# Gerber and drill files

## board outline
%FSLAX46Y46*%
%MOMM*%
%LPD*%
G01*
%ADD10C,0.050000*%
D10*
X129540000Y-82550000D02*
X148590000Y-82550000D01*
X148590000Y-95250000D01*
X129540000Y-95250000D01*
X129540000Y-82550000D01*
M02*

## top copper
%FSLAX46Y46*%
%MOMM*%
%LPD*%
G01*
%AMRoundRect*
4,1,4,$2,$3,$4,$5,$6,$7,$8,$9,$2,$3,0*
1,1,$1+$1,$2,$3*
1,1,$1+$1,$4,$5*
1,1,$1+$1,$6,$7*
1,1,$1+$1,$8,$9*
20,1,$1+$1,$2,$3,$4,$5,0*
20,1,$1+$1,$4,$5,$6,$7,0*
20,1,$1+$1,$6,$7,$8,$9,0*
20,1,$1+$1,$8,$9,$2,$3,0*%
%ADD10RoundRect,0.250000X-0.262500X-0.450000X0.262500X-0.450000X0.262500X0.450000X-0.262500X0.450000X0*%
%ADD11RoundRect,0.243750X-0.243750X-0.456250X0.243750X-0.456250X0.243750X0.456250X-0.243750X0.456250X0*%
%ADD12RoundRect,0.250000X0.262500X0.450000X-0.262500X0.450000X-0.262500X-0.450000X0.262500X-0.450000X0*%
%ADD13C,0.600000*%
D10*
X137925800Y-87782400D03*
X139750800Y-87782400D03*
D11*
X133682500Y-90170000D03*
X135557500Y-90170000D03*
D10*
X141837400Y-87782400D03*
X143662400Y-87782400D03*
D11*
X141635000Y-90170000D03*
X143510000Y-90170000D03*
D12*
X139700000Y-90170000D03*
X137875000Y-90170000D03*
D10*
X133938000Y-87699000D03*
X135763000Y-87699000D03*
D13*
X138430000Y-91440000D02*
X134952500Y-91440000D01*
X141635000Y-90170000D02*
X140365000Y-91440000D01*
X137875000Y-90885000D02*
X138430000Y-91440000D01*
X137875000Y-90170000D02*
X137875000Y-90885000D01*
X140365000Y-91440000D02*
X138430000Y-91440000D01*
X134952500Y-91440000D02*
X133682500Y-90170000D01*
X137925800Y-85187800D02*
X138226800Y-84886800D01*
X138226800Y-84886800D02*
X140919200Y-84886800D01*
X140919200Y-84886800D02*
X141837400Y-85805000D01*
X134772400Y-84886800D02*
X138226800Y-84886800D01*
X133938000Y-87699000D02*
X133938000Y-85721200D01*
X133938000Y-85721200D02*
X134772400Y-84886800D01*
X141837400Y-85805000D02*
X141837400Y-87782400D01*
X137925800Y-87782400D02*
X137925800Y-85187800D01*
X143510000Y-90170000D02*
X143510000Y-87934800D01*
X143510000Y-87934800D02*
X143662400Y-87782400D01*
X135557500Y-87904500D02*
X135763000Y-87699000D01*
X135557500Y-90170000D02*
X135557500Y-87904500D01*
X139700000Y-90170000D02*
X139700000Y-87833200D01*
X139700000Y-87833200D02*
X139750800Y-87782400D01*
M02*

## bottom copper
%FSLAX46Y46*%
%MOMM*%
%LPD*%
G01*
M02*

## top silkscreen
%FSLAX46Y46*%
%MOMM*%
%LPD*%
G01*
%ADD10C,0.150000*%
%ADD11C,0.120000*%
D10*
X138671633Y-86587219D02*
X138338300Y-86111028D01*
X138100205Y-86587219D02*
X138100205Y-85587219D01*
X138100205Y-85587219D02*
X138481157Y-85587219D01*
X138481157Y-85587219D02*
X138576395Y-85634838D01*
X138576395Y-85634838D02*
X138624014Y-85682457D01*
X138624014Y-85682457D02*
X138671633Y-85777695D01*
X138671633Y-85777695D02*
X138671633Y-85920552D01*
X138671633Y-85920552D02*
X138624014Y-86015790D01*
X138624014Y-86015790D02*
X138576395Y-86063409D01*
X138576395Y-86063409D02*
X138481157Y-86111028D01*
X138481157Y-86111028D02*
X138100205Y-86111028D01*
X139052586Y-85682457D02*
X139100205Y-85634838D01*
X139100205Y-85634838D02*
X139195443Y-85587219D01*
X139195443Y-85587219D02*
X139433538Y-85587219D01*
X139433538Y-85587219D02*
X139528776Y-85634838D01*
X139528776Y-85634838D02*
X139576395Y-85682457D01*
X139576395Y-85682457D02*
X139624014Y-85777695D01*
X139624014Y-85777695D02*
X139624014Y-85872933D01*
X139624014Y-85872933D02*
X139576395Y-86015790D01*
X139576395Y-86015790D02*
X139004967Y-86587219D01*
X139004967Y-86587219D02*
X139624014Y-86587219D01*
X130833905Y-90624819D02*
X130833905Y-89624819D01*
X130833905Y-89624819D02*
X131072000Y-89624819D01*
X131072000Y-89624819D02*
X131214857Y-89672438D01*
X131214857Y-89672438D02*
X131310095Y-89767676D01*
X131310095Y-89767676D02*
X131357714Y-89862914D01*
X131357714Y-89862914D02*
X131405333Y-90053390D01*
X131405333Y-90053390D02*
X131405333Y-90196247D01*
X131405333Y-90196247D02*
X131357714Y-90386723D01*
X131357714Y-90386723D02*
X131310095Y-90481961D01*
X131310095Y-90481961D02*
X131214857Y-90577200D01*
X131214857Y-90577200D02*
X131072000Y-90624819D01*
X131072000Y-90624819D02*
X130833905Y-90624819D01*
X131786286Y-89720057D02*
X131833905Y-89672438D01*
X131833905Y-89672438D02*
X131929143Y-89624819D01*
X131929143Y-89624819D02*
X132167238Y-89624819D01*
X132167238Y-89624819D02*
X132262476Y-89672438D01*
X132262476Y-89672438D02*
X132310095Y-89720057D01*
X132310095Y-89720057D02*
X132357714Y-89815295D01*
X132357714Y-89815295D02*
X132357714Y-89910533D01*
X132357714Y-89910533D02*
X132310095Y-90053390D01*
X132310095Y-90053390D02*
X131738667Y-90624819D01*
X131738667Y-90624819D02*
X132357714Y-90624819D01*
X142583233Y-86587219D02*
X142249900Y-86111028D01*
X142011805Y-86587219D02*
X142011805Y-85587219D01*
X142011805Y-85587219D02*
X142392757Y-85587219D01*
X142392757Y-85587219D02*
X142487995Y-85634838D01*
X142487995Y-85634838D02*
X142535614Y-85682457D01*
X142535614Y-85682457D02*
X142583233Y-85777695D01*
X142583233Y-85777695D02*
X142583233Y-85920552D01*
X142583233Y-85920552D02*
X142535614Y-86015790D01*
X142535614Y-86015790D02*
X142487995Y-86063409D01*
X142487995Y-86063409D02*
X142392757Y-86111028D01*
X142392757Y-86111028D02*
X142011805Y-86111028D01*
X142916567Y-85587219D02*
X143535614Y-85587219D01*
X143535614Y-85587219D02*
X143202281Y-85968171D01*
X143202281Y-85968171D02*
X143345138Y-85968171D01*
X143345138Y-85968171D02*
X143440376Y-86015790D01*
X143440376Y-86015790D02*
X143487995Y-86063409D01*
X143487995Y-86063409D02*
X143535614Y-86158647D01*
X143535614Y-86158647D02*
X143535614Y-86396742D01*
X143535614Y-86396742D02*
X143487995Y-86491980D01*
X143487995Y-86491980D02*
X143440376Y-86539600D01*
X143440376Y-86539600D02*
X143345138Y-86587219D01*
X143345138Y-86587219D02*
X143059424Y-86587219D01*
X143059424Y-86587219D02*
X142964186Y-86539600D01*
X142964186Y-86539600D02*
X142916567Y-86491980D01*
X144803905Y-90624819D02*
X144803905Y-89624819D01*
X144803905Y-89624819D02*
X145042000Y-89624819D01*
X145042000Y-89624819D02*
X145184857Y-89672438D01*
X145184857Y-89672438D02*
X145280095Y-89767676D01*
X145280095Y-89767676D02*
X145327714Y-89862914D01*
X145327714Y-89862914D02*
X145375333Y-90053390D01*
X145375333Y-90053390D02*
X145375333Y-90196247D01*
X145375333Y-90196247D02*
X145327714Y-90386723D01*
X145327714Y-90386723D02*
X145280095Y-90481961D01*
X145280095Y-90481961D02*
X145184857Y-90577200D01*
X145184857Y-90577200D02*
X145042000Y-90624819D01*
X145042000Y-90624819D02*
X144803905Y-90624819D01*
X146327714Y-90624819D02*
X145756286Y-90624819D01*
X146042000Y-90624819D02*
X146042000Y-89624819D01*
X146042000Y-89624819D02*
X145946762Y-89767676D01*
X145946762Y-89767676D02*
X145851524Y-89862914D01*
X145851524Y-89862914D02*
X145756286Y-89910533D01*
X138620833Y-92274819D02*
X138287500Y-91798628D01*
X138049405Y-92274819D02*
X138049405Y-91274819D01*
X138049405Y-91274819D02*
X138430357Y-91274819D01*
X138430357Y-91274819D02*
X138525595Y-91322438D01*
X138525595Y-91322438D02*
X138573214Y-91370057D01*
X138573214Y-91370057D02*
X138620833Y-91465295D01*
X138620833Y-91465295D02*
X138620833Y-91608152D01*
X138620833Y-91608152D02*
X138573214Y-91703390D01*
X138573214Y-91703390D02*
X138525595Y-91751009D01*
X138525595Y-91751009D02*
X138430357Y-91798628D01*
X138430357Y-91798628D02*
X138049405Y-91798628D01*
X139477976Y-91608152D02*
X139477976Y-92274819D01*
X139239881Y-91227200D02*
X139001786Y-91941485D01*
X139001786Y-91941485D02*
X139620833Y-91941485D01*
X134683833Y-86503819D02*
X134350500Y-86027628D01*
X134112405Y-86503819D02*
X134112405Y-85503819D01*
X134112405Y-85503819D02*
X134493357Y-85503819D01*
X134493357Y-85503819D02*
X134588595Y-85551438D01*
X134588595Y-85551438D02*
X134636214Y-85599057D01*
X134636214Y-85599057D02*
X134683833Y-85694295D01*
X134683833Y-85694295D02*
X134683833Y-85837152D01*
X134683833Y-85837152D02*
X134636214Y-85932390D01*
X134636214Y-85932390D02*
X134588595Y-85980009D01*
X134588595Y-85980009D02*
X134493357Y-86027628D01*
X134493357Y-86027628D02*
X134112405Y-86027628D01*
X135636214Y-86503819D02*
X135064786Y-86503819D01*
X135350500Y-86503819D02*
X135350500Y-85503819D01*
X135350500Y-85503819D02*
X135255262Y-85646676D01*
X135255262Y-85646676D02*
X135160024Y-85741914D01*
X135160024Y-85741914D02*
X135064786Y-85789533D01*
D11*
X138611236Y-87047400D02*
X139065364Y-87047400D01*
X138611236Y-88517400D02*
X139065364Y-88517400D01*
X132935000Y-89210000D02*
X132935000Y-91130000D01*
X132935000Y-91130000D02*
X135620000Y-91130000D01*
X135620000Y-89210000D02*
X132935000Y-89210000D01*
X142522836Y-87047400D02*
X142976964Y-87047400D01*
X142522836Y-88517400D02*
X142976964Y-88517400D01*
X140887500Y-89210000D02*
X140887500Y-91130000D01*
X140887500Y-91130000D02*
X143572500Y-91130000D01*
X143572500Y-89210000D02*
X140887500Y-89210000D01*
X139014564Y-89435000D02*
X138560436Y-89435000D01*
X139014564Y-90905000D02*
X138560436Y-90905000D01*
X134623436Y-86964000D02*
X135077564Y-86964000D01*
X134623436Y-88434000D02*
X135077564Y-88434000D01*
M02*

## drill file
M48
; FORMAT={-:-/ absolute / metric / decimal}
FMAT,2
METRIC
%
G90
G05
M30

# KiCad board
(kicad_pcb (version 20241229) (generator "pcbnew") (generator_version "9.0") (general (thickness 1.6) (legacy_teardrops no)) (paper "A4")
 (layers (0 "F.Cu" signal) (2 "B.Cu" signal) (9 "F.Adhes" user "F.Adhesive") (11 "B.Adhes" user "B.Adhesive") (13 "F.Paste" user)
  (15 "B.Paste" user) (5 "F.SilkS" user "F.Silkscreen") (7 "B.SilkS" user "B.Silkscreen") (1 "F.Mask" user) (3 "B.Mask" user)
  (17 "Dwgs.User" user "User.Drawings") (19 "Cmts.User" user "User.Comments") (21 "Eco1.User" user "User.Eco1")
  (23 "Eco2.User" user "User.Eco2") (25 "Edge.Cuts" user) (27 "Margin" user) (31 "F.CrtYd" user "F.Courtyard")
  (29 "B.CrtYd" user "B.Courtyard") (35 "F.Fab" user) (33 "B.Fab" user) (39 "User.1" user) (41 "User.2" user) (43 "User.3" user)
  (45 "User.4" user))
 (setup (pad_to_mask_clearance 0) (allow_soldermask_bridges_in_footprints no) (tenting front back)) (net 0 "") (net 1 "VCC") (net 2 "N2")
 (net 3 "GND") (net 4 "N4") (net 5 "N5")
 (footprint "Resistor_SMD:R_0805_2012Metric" (layer "F.Cu") (at 138.8383 87.7824)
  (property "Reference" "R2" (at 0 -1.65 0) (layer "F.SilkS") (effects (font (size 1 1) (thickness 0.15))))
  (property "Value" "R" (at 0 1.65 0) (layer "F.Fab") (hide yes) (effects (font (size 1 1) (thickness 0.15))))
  (fp_line (start -0.227064 -0.735) (end 0.227064 -0.735) (stroke (width 0.12) (type solid)) (layer "F.SilkS"))
  (fp_line (start -0.227064 0.735) (end 0.227064 0.735) (stroke (width 0.12) (type solid)) (layer "F.SilkS"))
  (pad "1" smd roundrect (at -0.9125 0) (size 1.025 1.4) (layers "F.Cu" "F.Mask" "F.Paste") (roundrect_rratio 0.243902) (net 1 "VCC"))
  (pad "2" smd roundrect (at 0.9125 0) (size 1.025 1.4) (layers "F.Cu" "F.Mask" "F.Paste") (roundrect_rratio 0.243902) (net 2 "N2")))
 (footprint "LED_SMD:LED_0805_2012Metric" (layer "F.Cu") (at 134.62 90.17)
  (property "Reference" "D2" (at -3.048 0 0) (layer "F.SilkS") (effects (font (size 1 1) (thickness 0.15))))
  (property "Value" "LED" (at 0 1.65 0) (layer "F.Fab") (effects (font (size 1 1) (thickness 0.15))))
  (fp_line (start -1.685 -0.96) (end -1.685 0.96) (stroke (width 0.12) (type solid)) (layer "F.SilkS"))
  (fp_line (start -1.685 0.96) (end 1 0.96) (stroke (width 0.12) (type solid)) (layer "F.SilkS"))
  (fp_line (start 1 -0.96) (end -1.685 -0.96) (stroke (width 0.12) (type solid)) (layer "F.SilkS"))
  (pad "1" smd roundrect (at -0.9375 0) (size 0.975 1.4) (layers "F.Cu" "F.Mask" "F.Paste") (roundrect_rratio 0.25) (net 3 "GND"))
  (pad "2" smd roundrect (at 0.9375 0) (size 0.975 1.4) (layers "F.Cu" "F.Mask" "F.Paste") (roundrect_rratio 0.25) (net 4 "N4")))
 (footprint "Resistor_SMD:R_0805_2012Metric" (layer "F.Cu") (at 142.7499 87.7824)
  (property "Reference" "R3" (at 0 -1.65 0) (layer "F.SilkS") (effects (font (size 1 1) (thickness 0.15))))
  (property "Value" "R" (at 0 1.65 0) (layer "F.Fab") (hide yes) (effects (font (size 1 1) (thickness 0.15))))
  (fp_line (start -0.227064 -0.735) (end 0.227064 -0.735) (stroke (width 0.12) (type solid)) (layer "F.SilkS"))
  (fp_line (start -0.227064 0.735) (end 0.227064 0.735) (stroke (width 0.12) (type solid)) (layer "F.SilkS"))
  (pad "1" smd roundrect (at -0.9125 0) (size 1.025 1.4) (layers "F.Cu" "F.Mask" "F.Paste") (roundrect_rratio 0.243902) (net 1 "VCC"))
  (pad "2" smd roundrect (at 0.9125 0) (size 1.025 1.4) (layers "F.Cu" "F.Mask" "F.Paste") (roundrect_rratio 0.243902) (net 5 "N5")))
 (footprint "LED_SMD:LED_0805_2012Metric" (layer "F.Cu") (at 142.5725 90.17)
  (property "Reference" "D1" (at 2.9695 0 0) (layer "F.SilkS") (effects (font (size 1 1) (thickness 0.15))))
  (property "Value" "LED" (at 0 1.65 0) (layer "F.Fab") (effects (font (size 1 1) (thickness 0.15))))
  (fp_line (start -1.685 -0.96) (end -1.685 0.96) (stroke (width 0.12) (type solid)) (layer "F.SilkS"))
  (fp_line (start -1.685 0.96) (end 1 0.96) (stroke (width 0.12) (type solid)) (layer "F.SilkS"))
  (fp_line (start 1 -0.96) (end -1.685 -0.96) (stroke (width 0.12) (type solid)) (layer "F.SilkS"))
  (pad "1" smd roundrect (at -0.9375 0) (size 0.975 1.4) (layers "F.Cu" "F.Mask" "F.Paste") (roundrect_rratio 0.25) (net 3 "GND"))
  (pad "2" smd roundrect (at 0.9375 0) (size 0.975 1.4) (layers "F.Cu" "F.Mask" "F.Paste") (roundrect_rratio 0.25) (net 5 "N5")))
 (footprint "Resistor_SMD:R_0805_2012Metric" (layer "F.Cu") (at 138.7875 90.17 180)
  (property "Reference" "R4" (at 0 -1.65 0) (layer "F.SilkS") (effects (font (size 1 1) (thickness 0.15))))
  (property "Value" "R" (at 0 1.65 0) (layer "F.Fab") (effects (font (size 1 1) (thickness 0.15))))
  (fp_line (start -0.227064 0.735) (end 0.227064 0.735) (stroke (width 0.12) (type solid)) (layer "F.SilkS"))
  (fp_line (start -0.227064 -0.735) (end 0.227064 -0.735) (stroke (width 0.12) (type solid)) (layer "F.SilkS"))
  (pad "1" smd roundrect (at -0.9125 0 180) (size 1.025 1.4) (layers "F.Cu" "F.Mask" "F.Paste") (roundrect_rratio 0.243902) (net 2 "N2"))
  (pad "2" smd roundrect (at 0.9125 0 180) (size 1.025 1.4) (layers "F.Cu" "F.Mask" "F.Paste") (roundrect_rratio 0.243902) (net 3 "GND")))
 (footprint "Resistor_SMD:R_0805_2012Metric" (layer "F.Cu") (at 134.8505 87.699)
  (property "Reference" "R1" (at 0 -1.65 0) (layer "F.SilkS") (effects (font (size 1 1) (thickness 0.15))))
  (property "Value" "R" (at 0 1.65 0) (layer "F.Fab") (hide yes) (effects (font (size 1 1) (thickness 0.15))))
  (fp_line (start -0.227064 -0.735) (end 0.227064 -0.735) (stroke (width 0.12) (type solid)) (layer "F.SilkS"))
  (fp_line (start -0.227064 0.735) (end 0.227064 0.735) (stroke (width 0.12) (type solid)) (layer "F.SilkS"))
  (pad "1" smd roundrect (at -0.9125 0) (size 1.025 1.4) (layers "F.Cu" "F.Mask" "F.Paste") (roundrect_rratio 0.243902) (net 1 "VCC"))
  (pad "2" smd roundrect (at 0.9125 0) (size 1.025 1.4) (layers "F.Cu" "F.Mask" "F.Paste") (roundrect_rratio 0.243902) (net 4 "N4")))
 (gr_rect (start 129.54 82.55) (end 148.59 95.25) (stroke (width 0.05) (type default)) (fill no) (layer "Edge.Cuts"))
 (segment (start 138.43 91.44) (end 134.9525 91.44) (width 0.6) (layer "F.Cu") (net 3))
 (segment (start 141.635 90.17) (end 140.365 91.44) (width 0.6) (layer "F.Cu") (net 3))
 (segment (start 137.875 90.885) (end 138.43 91.44) (width 0.6) (layer "F.Cu") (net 3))
 (segment (start 137.875 90.17) (end 137.875 90.885) (width 0.6) (layer "F.Cu") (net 3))
 (segment (start 140.365 91.44) (end 138.43 91.44) (width 0.6) (layer "F.Cu") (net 3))
 (segment (start 134.9525 91.44) (end 133.6825 90.17) (width 0.6) (layer "F.Cu") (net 3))
 (segment (start 137.9258 85.1878) (end 138.2268 84.8868) (width 0.6) (layer "F.Cu") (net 1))
 (segment (start 138.2268 84.8868) (end 140.9192 84.8868) (width 0.6) (layer "F.Cu") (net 1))
 (segment (start 140.9192 84.8868) (end 141.8374 85.805) (width 0.6) (layer "F.Cu") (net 1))
 (segment (start 134.7724 84.8868) (end 138.2268 84.8868) (width 0.6) (layer "F.Cu") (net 1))
 (segment (start 133.938 87.699) (end 133.938 85.7212) (width 0.6) (layer "F.Cu") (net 1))
 (segment (start 133.938 85.7212) (end 134.7724 84.8868) (width 0.6) (layer "F.Cu") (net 1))
 (segment (start 141.8374 85.805) (end 141.8374 87.7824) (width 0.6) (layer "F.Cu") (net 1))
 (segment (start 137.9258 87.7824) (end 137.9258 85.1878) (width 0.6) (layer "F.Cu") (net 1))
 (segment (start 143.51 90.17) (end 143.51 87.9348) (width 0.6) (layer "F.Cu") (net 5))
 (segment (start 143.51 87.9348) (end 143.6624 87.7824) (width 0.6) (layer "F.Cu") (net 5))
 (segment (start 135.5575 87.9045) (end 135.763 87.699) (width 0.6) (layer "F.Cu") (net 4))
 (segment (start 135.5575 90.17) (end 135.5575 87.9045) (width 0.6) (layer "F.Cu") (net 4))
 (segment (start 139.7 90.17) (end 139.7 87.8332) (width 0.6) (layer "F.Cu") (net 2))
 (segment (start 139.7 87.8332) (end 139.7508 87.7824) (width 0.6) (layer "F.Cu") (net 2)))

